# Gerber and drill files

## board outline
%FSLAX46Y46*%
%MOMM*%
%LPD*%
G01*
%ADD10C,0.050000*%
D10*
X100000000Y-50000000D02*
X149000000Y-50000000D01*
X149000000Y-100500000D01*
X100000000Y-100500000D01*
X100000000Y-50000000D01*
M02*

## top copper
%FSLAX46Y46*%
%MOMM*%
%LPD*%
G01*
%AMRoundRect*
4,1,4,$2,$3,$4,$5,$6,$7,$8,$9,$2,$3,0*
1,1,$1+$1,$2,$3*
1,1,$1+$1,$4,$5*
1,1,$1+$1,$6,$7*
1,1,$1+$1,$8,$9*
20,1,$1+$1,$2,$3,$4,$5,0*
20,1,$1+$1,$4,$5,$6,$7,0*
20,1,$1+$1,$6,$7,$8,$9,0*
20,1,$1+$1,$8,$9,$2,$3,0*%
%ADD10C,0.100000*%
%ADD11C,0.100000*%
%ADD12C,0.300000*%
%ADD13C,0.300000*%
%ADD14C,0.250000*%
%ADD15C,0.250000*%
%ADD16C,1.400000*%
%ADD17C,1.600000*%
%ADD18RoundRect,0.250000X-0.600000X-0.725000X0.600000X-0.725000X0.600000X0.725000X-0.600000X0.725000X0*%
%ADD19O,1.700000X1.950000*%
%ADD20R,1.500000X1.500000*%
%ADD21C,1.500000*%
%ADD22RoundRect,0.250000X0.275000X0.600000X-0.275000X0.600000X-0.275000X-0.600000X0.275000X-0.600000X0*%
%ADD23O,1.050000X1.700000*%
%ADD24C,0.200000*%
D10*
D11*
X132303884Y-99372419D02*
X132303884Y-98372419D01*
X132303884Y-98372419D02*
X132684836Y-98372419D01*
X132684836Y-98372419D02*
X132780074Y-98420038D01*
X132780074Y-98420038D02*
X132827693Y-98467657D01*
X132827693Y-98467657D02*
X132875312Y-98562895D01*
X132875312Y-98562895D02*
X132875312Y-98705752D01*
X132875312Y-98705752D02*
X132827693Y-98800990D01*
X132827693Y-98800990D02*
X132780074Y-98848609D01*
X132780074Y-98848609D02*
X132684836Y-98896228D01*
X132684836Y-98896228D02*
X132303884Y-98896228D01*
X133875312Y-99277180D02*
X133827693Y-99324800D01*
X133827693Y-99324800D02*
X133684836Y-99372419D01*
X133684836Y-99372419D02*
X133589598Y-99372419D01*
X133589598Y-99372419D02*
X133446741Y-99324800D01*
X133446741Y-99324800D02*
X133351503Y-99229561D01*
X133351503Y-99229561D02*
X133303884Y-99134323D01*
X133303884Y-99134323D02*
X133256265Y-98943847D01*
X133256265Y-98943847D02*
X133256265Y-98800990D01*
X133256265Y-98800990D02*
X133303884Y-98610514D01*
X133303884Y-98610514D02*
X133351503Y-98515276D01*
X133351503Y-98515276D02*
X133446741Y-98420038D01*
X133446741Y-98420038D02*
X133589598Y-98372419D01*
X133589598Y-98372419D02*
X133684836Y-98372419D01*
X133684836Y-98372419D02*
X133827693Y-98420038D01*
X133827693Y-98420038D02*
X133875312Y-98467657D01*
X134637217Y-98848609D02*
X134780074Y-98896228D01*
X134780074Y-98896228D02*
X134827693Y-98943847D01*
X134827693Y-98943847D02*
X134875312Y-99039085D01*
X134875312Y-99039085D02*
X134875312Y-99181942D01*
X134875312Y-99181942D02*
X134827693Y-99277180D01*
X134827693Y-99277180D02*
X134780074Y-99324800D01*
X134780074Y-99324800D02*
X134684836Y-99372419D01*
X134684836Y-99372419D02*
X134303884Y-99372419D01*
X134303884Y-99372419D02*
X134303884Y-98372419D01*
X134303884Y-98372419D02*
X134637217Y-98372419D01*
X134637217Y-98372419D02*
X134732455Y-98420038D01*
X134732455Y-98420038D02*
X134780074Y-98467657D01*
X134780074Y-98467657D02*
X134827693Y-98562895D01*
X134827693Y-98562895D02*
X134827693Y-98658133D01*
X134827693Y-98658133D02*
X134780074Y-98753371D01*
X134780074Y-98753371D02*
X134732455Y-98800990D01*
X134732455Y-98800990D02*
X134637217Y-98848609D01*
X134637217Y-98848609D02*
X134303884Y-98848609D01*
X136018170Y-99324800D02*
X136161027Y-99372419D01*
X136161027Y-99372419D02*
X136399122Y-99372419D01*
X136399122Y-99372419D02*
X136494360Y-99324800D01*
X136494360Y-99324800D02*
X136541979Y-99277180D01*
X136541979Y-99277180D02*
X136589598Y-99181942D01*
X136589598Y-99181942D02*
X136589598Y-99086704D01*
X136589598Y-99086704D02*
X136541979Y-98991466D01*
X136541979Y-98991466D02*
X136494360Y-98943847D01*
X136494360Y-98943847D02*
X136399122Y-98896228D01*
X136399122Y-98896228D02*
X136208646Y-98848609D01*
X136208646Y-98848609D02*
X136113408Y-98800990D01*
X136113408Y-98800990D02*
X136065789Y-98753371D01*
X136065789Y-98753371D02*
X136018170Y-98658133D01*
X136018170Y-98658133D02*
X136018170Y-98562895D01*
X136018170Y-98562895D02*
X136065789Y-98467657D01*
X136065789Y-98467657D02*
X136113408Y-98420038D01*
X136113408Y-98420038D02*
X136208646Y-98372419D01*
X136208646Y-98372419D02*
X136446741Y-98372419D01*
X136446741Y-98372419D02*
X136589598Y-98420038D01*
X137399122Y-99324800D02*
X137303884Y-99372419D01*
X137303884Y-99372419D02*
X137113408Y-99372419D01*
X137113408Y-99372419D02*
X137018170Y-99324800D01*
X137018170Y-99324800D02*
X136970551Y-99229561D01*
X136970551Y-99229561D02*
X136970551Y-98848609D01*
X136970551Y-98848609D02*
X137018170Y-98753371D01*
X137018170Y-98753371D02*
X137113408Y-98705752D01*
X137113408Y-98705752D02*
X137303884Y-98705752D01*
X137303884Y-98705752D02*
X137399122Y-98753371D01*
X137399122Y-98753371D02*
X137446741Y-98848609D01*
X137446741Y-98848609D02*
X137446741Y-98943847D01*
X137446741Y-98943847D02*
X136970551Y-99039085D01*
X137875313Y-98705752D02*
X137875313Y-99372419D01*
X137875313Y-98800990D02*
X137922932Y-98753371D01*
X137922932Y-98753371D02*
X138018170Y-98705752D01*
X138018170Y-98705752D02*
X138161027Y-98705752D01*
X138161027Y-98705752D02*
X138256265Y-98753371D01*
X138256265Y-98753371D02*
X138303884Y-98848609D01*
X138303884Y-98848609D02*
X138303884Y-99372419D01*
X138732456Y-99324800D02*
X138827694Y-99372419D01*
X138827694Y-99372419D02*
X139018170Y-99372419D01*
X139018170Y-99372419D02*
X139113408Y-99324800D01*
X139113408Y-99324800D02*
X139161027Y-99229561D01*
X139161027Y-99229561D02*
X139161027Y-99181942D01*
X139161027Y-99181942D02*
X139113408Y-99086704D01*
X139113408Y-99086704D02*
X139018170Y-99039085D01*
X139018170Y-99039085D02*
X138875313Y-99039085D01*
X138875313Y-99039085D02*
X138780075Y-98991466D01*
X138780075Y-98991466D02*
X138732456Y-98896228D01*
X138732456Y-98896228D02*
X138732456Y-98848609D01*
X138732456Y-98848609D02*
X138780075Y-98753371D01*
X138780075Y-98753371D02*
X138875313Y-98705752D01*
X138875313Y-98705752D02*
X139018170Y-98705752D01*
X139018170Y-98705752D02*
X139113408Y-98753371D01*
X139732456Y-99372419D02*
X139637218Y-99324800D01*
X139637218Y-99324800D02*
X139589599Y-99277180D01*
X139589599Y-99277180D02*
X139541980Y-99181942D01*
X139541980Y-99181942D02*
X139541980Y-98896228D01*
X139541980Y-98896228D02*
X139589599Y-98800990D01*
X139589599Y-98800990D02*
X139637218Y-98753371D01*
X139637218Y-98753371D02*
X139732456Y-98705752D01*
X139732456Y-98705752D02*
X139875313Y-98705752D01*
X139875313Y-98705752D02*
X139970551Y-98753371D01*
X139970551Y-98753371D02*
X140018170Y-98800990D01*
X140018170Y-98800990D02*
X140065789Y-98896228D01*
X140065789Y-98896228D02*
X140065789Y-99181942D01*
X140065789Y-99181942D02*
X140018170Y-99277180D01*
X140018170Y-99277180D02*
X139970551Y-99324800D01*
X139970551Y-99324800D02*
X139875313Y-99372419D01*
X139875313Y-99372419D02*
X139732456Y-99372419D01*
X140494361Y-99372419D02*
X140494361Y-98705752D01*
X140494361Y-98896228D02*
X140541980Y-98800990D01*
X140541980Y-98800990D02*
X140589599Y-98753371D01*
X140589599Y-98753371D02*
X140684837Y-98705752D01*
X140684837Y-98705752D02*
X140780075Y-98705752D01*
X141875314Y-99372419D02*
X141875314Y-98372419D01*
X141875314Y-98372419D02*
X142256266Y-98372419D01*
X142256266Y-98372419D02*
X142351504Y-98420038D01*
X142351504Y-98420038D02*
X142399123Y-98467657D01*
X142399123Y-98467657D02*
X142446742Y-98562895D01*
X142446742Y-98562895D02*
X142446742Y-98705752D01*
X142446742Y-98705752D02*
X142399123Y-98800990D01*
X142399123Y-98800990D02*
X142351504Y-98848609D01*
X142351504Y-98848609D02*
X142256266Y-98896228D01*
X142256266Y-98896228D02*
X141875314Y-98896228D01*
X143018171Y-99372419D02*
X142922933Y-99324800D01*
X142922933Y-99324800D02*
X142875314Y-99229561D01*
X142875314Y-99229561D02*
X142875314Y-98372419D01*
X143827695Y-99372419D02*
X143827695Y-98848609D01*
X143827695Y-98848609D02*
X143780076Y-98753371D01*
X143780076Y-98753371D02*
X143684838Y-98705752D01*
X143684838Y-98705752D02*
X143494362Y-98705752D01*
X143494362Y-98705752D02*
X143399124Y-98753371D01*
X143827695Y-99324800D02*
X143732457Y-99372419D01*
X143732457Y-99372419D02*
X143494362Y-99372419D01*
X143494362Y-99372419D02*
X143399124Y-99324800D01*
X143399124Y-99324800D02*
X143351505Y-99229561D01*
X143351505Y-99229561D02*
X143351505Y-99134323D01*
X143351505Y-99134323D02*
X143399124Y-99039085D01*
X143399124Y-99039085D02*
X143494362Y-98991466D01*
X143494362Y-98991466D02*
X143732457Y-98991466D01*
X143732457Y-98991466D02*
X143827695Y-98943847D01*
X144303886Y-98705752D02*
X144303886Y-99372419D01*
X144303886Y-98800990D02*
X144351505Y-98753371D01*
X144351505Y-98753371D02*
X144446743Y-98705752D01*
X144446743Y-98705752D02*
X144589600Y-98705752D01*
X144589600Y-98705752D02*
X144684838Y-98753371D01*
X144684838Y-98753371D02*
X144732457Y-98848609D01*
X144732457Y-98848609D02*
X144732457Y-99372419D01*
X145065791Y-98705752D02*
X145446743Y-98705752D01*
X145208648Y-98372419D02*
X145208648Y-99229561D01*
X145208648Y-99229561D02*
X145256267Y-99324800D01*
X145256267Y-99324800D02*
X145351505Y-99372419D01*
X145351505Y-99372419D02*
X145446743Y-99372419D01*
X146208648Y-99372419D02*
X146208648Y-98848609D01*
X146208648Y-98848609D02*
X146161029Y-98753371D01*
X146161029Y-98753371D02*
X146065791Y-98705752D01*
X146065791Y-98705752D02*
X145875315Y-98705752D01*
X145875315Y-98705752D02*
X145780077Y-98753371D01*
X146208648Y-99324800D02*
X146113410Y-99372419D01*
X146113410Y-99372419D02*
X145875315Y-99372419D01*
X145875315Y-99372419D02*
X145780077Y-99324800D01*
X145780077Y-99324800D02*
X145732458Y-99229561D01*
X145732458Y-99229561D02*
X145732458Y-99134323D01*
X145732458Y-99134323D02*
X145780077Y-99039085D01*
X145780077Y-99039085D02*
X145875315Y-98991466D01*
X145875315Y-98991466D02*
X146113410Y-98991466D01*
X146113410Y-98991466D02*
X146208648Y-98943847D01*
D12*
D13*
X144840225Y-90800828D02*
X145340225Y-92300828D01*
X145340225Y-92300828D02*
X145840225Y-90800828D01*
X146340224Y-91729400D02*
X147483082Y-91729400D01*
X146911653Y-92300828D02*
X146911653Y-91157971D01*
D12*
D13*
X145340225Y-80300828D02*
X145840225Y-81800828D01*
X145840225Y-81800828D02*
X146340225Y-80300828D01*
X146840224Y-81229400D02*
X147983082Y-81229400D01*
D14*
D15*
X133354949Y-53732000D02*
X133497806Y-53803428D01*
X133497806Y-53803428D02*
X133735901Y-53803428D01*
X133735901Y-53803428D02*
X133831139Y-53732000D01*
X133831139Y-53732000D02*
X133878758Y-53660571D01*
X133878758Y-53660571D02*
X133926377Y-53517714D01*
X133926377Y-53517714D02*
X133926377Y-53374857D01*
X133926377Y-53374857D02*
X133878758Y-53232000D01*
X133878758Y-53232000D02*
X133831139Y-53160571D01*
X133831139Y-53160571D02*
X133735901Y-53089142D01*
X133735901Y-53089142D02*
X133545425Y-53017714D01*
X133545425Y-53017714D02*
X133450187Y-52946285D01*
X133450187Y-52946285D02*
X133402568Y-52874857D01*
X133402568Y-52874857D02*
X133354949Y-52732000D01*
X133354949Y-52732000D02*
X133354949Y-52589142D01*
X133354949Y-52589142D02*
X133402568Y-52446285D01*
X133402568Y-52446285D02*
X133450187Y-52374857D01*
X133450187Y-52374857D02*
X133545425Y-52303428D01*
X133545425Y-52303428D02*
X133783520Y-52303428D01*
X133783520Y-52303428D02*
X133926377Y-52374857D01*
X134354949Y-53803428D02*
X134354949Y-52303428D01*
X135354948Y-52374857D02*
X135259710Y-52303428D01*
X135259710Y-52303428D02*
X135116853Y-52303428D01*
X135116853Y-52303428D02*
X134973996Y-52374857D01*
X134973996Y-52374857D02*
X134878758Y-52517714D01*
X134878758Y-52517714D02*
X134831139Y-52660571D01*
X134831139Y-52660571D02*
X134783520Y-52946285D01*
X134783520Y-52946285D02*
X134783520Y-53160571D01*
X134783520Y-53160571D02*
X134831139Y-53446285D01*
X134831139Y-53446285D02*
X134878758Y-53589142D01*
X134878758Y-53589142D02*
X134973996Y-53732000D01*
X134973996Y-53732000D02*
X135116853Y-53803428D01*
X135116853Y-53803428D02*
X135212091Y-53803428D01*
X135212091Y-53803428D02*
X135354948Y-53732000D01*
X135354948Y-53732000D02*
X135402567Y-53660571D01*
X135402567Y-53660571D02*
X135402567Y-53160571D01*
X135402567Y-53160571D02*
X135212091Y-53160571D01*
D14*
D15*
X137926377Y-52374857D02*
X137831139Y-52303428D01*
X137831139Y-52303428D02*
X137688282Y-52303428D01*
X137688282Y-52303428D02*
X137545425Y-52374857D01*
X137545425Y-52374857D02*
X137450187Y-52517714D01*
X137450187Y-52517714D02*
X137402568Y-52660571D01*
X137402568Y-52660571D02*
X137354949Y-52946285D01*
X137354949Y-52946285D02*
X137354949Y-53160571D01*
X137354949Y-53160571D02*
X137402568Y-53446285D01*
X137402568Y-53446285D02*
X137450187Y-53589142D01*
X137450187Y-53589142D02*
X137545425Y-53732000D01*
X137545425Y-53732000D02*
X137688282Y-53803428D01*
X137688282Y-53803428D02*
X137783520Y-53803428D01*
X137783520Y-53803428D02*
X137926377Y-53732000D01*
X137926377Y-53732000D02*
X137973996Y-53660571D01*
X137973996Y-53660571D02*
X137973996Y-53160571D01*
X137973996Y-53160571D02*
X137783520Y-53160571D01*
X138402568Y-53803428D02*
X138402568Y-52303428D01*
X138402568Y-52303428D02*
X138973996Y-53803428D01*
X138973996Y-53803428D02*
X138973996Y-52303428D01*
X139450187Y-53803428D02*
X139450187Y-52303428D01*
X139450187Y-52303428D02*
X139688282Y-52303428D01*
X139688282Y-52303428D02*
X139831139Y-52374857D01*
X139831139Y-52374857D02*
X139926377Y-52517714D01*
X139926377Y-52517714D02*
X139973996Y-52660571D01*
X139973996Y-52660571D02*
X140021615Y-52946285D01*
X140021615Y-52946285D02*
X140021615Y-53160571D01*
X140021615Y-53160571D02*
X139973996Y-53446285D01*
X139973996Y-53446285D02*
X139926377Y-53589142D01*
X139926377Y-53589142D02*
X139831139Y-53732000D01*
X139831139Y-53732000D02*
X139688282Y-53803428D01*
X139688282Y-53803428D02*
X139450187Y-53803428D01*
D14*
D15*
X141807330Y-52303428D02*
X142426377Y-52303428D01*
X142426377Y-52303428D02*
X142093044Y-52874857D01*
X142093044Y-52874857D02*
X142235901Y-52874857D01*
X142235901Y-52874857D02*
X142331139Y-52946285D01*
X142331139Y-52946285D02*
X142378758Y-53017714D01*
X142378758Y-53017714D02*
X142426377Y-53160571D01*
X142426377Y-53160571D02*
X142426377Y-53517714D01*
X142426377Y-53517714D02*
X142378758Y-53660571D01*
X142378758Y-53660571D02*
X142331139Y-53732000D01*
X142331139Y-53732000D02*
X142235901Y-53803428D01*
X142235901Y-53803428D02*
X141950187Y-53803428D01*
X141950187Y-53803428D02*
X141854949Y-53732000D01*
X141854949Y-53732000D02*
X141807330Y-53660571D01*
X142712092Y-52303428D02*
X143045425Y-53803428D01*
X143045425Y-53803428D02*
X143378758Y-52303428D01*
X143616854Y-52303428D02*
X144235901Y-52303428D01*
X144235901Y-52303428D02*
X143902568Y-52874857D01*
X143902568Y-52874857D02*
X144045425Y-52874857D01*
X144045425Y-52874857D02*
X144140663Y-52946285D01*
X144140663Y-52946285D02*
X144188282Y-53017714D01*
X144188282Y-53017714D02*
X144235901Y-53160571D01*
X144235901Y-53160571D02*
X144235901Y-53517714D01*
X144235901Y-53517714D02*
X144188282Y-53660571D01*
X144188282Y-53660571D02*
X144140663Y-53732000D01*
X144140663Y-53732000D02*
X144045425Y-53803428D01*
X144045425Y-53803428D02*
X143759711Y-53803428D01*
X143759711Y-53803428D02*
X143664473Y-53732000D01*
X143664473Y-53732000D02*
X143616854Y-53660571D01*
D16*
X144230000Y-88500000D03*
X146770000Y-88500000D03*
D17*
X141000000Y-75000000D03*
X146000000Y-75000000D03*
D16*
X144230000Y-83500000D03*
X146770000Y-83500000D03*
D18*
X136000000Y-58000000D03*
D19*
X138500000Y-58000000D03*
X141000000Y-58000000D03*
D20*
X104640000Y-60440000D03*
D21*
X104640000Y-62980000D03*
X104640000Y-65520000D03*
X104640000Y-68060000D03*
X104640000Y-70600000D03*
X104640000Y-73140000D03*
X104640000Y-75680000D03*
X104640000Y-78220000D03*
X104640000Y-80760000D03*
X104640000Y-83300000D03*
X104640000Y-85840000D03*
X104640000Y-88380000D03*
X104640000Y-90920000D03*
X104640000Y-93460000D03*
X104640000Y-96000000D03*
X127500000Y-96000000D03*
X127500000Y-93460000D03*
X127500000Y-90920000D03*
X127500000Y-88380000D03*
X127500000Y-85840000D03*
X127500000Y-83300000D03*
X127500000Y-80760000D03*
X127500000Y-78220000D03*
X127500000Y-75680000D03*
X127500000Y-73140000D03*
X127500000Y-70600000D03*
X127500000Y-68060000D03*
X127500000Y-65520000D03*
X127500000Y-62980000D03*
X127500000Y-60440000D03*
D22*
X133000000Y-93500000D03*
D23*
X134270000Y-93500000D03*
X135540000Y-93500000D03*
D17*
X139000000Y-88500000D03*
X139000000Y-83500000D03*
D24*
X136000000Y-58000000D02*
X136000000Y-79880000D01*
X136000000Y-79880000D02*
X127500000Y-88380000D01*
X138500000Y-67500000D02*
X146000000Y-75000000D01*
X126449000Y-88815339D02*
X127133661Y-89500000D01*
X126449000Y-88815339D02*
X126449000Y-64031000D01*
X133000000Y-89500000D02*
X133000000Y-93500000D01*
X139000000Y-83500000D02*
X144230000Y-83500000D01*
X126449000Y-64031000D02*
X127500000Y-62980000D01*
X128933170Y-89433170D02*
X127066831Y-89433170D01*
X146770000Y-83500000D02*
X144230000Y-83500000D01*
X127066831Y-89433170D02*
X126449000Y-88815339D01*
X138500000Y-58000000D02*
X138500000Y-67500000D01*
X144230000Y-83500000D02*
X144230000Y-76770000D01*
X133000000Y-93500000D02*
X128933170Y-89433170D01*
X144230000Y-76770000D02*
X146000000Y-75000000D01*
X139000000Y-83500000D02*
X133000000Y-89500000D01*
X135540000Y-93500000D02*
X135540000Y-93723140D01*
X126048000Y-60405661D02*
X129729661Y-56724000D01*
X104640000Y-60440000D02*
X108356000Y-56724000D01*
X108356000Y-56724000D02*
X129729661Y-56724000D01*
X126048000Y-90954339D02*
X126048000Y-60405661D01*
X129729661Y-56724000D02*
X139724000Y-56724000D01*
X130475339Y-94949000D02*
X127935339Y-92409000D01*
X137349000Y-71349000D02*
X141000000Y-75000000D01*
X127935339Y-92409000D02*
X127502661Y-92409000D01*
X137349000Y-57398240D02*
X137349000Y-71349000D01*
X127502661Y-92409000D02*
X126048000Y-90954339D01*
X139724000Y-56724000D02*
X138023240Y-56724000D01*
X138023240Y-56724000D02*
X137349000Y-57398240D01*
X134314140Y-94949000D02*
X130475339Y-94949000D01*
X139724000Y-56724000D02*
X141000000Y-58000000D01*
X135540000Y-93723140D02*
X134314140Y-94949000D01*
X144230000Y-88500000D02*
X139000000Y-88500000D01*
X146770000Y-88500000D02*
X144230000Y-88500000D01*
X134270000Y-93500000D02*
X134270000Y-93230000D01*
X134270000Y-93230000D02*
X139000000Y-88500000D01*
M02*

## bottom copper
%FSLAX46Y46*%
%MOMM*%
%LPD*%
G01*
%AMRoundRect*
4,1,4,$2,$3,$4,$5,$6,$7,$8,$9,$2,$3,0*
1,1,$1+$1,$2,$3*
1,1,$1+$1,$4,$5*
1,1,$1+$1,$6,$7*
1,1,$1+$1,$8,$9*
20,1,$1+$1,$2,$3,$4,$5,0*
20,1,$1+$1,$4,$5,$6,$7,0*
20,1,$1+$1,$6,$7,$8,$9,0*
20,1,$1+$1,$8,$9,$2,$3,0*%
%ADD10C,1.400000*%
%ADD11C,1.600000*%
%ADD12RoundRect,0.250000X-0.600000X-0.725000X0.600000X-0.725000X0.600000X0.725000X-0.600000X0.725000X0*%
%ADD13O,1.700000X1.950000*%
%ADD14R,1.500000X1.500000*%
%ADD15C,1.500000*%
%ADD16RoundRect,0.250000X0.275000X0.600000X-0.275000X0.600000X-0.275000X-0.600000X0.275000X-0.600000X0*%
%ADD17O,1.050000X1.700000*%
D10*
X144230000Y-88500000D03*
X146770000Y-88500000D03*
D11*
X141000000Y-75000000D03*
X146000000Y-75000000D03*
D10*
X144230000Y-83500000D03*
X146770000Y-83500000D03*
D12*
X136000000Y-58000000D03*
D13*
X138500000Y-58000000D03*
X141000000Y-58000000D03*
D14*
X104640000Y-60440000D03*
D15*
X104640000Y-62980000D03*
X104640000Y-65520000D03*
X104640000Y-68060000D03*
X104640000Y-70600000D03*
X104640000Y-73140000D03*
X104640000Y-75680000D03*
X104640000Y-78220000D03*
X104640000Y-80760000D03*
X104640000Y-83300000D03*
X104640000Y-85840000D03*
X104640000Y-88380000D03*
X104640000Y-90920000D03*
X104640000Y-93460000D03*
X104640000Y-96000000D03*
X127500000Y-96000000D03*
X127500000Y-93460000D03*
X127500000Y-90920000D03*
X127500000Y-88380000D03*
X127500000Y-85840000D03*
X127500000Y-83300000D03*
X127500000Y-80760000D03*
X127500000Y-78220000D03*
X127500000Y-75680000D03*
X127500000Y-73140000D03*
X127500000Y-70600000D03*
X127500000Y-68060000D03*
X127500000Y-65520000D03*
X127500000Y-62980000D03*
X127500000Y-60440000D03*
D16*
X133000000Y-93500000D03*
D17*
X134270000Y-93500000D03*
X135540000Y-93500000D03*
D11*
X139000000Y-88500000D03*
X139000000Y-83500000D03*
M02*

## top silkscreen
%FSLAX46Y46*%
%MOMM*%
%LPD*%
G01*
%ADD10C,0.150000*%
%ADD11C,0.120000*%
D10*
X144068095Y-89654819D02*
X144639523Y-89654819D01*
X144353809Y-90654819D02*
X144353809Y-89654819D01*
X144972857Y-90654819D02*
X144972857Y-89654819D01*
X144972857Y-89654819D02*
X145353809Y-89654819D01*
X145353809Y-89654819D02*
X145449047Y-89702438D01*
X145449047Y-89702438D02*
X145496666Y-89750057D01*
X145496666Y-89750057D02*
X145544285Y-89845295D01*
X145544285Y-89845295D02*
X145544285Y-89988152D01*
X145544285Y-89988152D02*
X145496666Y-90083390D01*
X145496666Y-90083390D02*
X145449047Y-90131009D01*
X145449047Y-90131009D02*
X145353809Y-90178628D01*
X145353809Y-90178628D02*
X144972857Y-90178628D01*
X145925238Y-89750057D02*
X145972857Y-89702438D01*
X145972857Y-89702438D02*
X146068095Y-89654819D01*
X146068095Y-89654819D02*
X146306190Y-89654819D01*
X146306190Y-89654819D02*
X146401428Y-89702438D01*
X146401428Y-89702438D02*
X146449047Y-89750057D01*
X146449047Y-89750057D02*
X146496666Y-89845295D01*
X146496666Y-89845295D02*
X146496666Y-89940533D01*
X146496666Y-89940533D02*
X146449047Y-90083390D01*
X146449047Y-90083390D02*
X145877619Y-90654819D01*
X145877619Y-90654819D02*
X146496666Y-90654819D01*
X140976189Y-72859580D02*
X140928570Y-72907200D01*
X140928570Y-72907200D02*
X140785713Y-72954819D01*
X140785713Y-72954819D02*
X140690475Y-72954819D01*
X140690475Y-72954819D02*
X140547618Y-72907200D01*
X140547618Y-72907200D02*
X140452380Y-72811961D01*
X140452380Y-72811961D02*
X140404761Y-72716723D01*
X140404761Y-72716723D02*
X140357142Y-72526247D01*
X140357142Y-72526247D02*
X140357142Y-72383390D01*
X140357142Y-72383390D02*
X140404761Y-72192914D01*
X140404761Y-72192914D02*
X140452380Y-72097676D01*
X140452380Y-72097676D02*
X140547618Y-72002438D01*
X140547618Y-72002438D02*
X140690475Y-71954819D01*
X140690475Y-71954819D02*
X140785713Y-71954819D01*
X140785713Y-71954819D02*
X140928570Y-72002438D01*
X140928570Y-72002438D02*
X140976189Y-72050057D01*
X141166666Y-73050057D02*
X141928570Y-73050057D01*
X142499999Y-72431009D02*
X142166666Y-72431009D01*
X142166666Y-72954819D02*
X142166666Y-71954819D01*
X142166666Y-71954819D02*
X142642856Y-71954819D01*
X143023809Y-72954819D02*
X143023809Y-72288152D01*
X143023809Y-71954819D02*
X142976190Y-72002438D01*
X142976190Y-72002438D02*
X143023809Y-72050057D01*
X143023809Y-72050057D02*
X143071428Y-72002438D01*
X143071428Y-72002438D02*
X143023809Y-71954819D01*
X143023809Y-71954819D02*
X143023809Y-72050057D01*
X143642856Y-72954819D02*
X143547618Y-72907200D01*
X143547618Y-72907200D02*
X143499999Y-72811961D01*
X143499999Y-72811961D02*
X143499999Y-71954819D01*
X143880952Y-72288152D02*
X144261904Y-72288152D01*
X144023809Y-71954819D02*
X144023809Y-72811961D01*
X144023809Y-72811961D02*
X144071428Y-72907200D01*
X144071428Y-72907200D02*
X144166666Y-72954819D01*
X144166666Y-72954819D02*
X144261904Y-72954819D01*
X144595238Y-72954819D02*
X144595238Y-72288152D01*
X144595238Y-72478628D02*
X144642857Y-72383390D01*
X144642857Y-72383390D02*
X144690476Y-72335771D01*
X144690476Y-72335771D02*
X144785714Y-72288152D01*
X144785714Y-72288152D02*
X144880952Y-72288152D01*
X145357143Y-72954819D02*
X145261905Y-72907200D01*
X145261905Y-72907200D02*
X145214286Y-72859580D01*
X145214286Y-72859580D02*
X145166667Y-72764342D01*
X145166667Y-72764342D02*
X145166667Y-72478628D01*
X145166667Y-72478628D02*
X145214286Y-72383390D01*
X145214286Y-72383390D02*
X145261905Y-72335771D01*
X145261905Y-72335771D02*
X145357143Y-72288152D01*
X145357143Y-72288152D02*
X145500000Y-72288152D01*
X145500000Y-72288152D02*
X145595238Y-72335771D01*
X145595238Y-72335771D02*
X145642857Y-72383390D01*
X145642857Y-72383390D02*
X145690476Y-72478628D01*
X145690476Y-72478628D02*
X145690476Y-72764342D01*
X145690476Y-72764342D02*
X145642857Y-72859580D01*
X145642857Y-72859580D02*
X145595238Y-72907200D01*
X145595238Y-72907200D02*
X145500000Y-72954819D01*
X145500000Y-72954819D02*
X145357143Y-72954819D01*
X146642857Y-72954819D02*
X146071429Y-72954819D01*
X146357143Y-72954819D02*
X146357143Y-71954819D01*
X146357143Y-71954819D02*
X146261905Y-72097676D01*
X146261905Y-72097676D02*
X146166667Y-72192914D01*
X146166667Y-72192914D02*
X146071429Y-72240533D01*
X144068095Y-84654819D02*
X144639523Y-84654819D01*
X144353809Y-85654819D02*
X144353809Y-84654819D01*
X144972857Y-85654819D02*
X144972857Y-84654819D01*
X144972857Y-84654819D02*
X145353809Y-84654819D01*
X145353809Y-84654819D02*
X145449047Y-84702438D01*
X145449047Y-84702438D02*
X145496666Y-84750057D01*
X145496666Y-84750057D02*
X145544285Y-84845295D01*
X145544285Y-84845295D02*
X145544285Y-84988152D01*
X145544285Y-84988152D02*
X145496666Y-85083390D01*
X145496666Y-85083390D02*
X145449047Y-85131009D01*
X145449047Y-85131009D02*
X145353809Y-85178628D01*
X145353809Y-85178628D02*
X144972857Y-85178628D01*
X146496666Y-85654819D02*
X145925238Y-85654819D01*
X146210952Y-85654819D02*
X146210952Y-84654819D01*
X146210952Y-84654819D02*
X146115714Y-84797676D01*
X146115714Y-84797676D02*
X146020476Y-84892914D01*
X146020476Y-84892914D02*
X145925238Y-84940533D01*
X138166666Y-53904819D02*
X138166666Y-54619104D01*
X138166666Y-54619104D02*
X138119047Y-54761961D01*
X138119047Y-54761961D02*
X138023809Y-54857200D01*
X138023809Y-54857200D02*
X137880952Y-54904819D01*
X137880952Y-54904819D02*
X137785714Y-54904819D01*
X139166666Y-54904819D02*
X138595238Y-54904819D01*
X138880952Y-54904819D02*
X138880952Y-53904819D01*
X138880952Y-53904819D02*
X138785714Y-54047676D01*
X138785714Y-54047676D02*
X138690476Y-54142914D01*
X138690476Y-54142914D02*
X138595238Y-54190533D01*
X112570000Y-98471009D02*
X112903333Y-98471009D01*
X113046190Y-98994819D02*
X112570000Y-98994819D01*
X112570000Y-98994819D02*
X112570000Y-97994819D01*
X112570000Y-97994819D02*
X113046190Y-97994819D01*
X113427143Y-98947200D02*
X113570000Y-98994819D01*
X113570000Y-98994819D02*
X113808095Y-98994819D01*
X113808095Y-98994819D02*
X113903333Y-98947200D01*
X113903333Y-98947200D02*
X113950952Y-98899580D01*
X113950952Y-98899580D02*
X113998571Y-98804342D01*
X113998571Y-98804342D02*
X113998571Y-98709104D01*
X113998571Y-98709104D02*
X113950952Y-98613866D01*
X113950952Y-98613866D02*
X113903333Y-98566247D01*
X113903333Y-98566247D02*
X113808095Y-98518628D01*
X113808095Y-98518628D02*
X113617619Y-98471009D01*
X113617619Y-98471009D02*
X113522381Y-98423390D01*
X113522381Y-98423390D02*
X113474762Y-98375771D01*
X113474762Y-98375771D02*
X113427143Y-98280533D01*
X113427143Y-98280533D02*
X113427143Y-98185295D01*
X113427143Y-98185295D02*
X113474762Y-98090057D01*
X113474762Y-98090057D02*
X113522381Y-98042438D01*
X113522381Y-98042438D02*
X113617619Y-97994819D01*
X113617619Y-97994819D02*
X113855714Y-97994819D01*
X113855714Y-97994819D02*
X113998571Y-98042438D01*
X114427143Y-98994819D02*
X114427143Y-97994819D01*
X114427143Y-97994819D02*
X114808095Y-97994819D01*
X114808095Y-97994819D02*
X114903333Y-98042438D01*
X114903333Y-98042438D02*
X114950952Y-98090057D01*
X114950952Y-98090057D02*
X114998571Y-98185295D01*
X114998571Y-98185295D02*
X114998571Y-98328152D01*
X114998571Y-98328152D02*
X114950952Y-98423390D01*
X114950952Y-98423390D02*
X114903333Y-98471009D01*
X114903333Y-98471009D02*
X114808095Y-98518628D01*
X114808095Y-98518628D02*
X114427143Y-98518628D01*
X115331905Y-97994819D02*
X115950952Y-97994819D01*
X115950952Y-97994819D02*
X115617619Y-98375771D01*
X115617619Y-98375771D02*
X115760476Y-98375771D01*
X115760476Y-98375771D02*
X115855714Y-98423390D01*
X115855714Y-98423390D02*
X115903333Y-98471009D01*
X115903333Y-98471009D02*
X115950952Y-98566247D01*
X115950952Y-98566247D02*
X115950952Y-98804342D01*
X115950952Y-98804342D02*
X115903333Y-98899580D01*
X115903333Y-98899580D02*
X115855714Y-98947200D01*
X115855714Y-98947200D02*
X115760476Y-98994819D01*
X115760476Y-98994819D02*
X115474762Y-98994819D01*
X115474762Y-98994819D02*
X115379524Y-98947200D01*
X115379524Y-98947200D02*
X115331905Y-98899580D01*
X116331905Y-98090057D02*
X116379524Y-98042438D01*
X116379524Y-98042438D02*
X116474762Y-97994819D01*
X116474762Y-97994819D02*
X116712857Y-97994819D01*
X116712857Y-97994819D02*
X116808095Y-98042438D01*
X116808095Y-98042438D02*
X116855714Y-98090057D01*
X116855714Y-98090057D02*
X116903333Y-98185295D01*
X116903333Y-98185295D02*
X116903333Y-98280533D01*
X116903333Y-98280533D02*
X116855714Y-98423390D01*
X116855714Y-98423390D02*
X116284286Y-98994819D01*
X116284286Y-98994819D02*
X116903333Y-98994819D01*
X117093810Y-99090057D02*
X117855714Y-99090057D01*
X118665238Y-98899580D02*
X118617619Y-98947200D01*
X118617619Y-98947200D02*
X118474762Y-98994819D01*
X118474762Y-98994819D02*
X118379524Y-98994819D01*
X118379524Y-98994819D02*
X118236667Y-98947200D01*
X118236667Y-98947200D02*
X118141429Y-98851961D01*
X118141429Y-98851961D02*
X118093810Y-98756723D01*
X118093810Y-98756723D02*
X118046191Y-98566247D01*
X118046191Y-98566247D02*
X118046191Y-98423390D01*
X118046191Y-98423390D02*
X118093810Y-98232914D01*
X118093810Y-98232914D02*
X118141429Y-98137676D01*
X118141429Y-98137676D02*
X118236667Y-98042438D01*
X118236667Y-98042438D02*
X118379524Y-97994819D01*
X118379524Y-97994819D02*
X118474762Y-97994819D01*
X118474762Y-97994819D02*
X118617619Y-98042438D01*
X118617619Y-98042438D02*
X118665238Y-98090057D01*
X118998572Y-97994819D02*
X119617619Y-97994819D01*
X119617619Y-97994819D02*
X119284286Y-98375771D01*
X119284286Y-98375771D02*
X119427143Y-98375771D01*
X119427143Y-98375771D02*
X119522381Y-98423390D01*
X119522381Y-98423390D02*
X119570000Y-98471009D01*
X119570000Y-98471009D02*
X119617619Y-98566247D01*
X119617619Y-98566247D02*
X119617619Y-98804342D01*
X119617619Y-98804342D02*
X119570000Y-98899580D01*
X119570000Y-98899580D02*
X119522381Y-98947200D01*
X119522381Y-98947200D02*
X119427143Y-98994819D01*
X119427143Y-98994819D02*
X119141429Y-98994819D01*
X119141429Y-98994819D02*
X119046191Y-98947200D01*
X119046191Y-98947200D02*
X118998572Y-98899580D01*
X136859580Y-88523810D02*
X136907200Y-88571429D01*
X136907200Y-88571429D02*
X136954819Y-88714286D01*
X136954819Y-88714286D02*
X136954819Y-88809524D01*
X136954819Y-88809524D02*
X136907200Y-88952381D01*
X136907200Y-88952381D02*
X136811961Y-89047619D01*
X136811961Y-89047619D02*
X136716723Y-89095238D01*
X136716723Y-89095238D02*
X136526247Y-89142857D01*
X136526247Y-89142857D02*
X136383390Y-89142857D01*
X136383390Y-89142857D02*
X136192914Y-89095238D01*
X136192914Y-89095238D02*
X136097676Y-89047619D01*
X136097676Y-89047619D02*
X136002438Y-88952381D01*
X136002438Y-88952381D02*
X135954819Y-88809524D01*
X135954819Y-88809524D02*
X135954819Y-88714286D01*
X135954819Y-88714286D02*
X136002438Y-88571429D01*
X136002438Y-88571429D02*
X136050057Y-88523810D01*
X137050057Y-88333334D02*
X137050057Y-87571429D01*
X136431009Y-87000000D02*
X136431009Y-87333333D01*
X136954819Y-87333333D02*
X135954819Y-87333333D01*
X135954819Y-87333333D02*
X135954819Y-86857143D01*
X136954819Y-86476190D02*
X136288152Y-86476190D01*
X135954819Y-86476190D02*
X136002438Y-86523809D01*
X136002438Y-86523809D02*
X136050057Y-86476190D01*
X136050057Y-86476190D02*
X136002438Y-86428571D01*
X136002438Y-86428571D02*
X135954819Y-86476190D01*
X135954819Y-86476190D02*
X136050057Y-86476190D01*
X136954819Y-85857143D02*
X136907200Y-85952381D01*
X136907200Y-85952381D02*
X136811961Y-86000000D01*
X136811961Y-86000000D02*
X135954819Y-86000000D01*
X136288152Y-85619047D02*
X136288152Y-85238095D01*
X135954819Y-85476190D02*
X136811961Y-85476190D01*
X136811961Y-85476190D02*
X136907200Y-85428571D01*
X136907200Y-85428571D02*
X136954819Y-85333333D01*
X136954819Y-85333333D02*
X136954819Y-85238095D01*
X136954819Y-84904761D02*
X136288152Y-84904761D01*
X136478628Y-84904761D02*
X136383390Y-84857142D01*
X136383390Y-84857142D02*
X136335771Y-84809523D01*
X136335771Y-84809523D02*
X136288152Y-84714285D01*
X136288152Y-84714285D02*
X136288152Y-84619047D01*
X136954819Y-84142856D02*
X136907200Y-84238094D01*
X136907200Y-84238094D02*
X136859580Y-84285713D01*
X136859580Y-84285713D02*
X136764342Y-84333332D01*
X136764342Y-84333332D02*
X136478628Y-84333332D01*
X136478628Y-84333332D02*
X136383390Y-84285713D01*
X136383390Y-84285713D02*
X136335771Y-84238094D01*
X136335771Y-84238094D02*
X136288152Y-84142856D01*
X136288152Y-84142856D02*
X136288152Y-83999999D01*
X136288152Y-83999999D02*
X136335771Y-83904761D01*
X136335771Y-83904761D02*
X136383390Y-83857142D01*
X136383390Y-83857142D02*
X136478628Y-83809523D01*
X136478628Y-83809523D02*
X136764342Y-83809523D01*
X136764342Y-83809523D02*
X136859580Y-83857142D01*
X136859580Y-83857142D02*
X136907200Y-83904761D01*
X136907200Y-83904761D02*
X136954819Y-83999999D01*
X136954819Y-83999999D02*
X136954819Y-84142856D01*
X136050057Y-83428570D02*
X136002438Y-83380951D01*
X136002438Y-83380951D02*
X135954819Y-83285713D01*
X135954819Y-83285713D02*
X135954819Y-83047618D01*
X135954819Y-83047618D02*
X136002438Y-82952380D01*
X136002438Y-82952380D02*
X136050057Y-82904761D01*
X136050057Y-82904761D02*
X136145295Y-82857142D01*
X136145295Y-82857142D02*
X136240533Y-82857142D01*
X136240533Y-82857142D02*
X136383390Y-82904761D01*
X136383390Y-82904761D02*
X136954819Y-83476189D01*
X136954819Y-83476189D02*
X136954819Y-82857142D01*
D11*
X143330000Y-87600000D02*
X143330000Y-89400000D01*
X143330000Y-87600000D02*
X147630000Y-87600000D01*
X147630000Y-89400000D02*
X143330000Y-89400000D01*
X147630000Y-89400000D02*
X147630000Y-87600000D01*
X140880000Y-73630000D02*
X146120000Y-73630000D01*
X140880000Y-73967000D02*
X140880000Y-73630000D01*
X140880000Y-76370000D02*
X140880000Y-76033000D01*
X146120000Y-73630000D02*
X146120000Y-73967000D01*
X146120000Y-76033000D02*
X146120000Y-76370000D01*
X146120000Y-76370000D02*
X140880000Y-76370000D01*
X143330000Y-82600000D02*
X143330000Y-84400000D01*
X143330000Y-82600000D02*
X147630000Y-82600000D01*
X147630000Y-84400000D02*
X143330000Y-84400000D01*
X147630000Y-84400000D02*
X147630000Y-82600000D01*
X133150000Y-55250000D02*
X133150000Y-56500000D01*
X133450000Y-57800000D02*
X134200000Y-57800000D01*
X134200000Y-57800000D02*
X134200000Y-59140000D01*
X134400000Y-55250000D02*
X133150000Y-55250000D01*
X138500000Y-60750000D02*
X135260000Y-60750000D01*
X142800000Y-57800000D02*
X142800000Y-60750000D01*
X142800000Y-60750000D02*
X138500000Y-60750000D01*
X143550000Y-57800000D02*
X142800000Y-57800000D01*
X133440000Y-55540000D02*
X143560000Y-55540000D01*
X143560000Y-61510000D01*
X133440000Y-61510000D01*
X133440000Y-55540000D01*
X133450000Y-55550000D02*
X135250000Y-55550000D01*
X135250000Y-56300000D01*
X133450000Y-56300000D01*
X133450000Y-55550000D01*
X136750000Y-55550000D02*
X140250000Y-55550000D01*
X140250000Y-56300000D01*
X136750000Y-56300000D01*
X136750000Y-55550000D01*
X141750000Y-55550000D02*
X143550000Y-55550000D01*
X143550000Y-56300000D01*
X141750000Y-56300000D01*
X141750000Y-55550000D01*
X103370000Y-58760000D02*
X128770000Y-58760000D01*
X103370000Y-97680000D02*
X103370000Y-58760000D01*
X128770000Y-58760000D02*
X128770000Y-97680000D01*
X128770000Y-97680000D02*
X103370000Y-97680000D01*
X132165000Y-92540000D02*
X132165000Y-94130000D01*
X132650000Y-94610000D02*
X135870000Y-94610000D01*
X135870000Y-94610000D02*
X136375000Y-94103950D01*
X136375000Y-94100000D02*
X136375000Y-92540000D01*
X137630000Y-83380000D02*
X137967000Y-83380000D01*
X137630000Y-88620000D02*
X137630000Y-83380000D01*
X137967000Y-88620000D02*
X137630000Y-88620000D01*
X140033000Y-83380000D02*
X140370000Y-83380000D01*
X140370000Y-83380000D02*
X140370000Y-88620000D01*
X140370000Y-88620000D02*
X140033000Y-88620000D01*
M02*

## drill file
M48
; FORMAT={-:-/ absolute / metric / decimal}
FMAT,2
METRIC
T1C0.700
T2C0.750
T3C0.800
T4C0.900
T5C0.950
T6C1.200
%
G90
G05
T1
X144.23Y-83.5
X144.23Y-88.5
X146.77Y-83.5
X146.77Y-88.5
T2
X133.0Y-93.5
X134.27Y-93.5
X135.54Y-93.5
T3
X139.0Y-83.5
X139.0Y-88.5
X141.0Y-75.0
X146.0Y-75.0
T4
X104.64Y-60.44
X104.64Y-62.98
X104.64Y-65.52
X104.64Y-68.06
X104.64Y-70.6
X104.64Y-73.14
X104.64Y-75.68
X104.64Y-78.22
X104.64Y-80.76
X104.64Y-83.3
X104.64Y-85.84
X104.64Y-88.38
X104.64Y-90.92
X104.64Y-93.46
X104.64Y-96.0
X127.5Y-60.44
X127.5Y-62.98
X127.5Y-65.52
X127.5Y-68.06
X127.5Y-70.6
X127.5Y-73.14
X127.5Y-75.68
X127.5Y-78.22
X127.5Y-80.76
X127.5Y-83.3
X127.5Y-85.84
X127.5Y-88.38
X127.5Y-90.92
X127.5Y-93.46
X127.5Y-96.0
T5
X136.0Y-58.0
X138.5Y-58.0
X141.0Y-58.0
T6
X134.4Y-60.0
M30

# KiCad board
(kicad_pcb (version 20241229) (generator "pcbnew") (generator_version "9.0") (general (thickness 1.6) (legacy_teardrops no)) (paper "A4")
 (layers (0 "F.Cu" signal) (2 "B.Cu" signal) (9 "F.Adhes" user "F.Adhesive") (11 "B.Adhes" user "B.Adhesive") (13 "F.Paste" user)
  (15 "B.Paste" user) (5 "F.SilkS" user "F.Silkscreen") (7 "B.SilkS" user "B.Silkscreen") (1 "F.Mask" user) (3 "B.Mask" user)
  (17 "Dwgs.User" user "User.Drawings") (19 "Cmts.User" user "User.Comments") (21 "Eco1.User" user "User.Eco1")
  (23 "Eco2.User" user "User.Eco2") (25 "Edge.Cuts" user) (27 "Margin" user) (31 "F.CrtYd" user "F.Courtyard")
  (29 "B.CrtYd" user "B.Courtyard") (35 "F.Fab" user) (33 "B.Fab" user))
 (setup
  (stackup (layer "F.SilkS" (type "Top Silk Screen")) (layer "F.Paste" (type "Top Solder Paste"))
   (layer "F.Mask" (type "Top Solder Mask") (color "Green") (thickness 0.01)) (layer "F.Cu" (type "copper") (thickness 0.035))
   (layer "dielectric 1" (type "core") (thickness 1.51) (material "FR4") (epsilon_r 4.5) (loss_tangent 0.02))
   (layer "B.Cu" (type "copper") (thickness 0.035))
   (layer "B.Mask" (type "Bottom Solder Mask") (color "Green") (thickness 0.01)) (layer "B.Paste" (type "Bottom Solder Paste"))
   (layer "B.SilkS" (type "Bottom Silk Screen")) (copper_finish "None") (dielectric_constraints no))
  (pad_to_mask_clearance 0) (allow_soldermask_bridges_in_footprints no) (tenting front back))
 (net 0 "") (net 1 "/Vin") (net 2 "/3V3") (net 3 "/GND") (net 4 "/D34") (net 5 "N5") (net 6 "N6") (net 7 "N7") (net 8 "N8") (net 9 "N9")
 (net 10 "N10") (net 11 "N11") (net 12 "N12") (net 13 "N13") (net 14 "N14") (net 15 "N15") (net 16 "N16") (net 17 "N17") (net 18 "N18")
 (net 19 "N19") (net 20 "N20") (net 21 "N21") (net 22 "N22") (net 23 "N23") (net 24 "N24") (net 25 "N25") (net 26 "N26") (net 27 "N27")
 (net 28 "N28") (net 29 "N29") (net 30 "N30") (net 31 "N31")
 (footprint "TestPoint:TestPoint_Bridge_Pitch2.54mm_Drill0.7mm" (layer "F.Cu") (at 144.23 88.5)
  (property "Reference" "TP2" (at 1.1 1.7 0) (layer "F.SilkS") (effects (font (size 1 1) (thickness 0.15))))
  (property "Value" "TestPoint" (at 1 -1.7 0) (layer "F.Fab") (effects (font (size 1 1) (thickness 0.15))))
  (fp_line (start -0.9 -0.9) (end -0.9 0.9) (stroke (width 0.12) (type solid)) (layer "F.SilkS"))
  (fp_line (start -0.9 -0.9) (end 3.4 -0.9) (stroke (width 0.12) (type solid)) (layer "F.SilkS"))
  (fp_line (start 3.4 0.9) (end -0.9 0.9) (stroke (width 0.12) (type solid)) (layer "F.SilkS"))
  (fp_line (start 3.4 0.9) (end 3.4 -0.9) (stroke (width 0.12) (type solid)) (layer "F.SilkS"))
  (pad "1" thru_hole circle (at 0 0) (size 1.4 1.4) (drill 0.7) (layers "*.Cu" "*.Mask") (remove_unused_layers no) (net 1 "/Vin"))
  (pad "1" thru_hole circle (at 2.54 0) (size 1.4 1.4) (drill 0.7) (layers "*.Cu" "*.Mask") (remove_unused_layers no) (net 1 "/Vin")))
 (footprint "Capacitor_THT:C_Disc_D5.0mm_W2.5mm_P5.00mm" (layer "F.Cu") (at 141 75)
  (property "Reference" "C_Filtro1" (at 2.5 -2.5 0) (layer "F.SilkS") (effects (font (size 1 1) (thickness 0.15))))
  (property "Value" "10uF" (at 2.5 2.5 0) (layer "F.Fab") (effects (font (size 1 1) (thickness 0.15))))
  (fp_line (start -0.12 -1.37) (end 5.12 -1.37) (stroke (width 0.12) (type solid)) (layer "F.SilkS"))
  (fp_line (start -0.12 -1.033) (end -0.12 -1.37) (stroke (width 0.12) (type solid)) (layer "F.SilkS"))
  (fp_line (start -0.12 1.37) (end -0.12 1.033) (stroke (width 0.12) (type solid)) (layer "F.SilkS"))
  (fp_line (start 5.12 -1.37) (end 5.12 -1.033) (stroke (width 0.12) (type solid)) (layer "F.SilkS"))
  (fp_line (start 5.12 1.033) (end 5.12 1.37) (stroke (width 0.12) (type solid)) (layer "F.SilkS"))
  (fp_line (start 5.12 1.37) (end -0.12 1.37) (stroke (width 0.12) (type solid)) (layer "F.SilkS"))
  (pad "1" thru_hole circle (at 0 0) (size 1.6 1.6) (drill 0.8) (layers "*.Cu" "*.Mask") (remove_unused_layers no) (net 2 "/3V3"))
  (pad "2" thru_hole circle (at 5 0) (size 1.6 1.6) (drill 0.8) (layers "*.Cu" "*.Mask") (remove_unused_layers no) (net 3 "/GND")))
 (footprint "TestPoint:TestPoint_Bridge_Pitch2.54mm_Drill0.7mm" (layer "F.Cu") (at 144.23 83.5)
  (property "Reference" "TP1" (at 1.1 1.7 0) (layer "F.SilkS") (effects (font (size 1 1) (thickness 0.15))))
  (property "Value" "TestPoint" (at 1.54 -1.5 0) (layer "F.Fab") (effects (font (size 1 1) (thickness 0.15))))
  (fp_line (start -0.9 -0.9) (end -0.9 0.9) (stroke (width 0.12) (type solid)) (layer "F.SilkS"))
  (fp_line (start -0.9 -0.9) (end 3.4 -0.9) (stroke (width 0.12) (type solid)) (layer "F.SilkS"))
  (fp_line (start 3.4 0.9) (end -0.9 0.9) (stroke (width 0.12) (type solid)) (layer "F.SilkS"))
  (fp_line (start 3.4 0.9) (end 3.4 -0.9) (stroke (width 0.12) (type solid)) (layer "F.SilkS"))
  (pad "1" thru_hole circle (at 0 0) (size 1.4 1.4) (drill 0.7) (layers "*.Cu" "*.Mask") (remove_unused_layers no) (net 3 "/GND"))
  (pad "1" thru_hole circle (at 2.54 0) (size 1.4 1.4) (drill 0.7) (layers "*.Cu" "*.Mask") (remove_unused_layers no) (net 3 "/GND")))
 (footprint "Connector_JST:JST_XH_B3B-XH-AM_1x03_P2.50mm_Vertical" (layer "F.Cu") (at 136 58)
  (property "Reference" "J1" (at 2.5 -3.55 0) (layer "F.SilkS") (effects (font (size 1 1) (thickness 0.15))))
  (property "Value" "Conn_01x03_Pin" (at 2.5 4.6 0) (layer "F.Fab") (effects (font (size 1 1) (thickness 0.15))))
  (fp_line (start -2.85 -2.75) (end -2.85 -1.5) (stroke (width 0.12) (type solid)) (layer "F.SilkS"))
  (fp_line (start -2.55 -0.2) (end -1.8 -0.2) (stroke (width 0.12) (type solid)) (layer "F.SilkS"))
  (fp_line (start -1.8 -0.2) (end -1.8 1.14) (stroke (width 0.12) (type solid)) (layer "F.SilkS"))
  (fp_line (start -1.6 -2.75) (end -2.85 -2.75) (stroke (width 0.12) (type solid)) (layer "F.SilkS"))
  (fp_line (start 2.5 2.75) (end -0.74 2.75) (stroke (width 0.12) (type solid)) (layer "F.SilkS"))
  (fp_line (start 6.8 -0.2) (end 6.8 2.75) (stroke (width 0.12) (type solid)) (layer "F.SilkS"))
  (fp_line (start 6.8 2.75) (end 2.5 2.75) (stroke (width 0.12) (type solid)) (layer "F.SilkS"))
  (fp_line (start 7.55 -0.2) (end 6.8 -0.2) (stroke (width 0.12) (type solid)) (layer "F.SilkS"))
  (fp_rect (start -2.56 -2.46) (end 7.56 3.51) (stroke (width 0.12) (type solid)) (fill no) (layer "F.SilkS"))
  (fp_rect (start -2.55 -2.45) (end -0.75 -1.7) (stroke (width 0.12) (type solid)) (fill no) (layer "F.SilkS"))
  (fp_rect (start 0.75 -2.45) (end 4.25 -1.7) (stroke (width 0.12) (type solid)) (fill no) (layer "F.SilkS"))
  (fp_rect (start 5.75 -2.45) (end 7.55 -1.7) (stroke (width 0.12) (type solid)) (fill no) (layer "F.SilkS"))
  (pad "" np_thru_hole circle (at -1.6 2) (size 1.2 1.2) (drill 1.2) (layers "*.Cu" "*.Mask"))
  (pad "1" thru_hole roundrect (at 0 0) (size 1.7 1.95) (drill 0.95) (layers "*.Cu" "*.Mask") (remove_unused_layers no)
   (roundrect_rratio 0.147059) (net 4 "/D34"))
  (pad "2" thru_hole oval (at 2.5 0) (size 1.7 1.95) (drill 0.95) (layers "*.Cu" "*.Mask") (remove_unused_layers no) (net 3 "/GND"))
  (pad "3" thru_hole oval (at 5 0) (size 1.7 1.95) (drill 0.95) (layers "*.Cu" "*.Mask") (remove_unused_layers no) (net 2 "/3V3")))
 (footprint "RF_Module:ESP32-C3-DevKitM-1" (layer "F.Cu") (at 104.64 60.44)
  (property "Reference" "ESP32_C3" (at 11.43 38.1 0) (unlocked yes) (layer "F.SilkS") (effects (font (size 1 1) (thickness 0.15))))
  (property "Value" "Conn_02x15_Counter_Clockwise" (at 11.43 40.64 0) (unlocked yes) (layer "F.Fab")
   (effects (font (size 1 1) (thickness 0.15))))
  (fp_line (start -1.27 -1.68) (end 24.13 -1.68) (stroke (width 0.12) (type solid)) (layer "F.SilkS"))
  (fp_line (start -1.27 37.24) (end -1.27 -1.68) (stroke (width 0.12) (type solid)) (layer "F.SilkS"))
  (fp_line (start 24.13 -1.68) (end 24.13 37.24) (stroke (width 0.12) (type solid)) (layer "F.SilkS"))
  (fp_line (start 24.13 37.24) (end -1.27 37.24) (stroke (width 0.12) (type solid)) (layer "F.SilkS"))
  (pad "1" thru_hole rect (at 0 0) (size 1.5 1.5) (drill 0.9) (layers "*.Cu" "*.Mask") (remove_unused_layers yes) (keep_end_layers yes)
   (zone_layer_connections) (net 2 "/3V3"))
  (pad "2" thru_hole circle (at 0 2.54) (size 1.5 1.5) (drill 0.9) (layers "*.Cu" "*.Mask") (remove_unused_layers yes) (keep_end_layers yes)
   (zone_layer_connections) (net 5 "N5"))
  (pad "3" thru_hole circle (at 0 5.08) (size 1.5 1.5) (drill 0.9) (layers "*.Cu" "*.Mask") (remove_unused_layers yes) (keep_end_layers yes)
   (zone_layer_connections) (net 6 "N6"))
  (pad "4" thru_hole circle (at 0 7.62) (size 1.5 1.5) (drill 0.9) (layers "*.Cu" "*.Mask") (remove_unused_layers yes) (keep_end_layers yes)
   (zone_layer_connections) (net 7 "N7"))
  (pad "5" thru_hole circle (at 0 10.16) (size 1.5 1.5) (drill 0.9) (layers "*.Cu" "*.Mask") (remove_unused_layers yes)
   (keep_end_layers yes) (zone_layer_connections) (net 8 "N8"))
  (pad "6" thru_hole circle (at 0 12.7) (size 1.5 1.5) (drill 0.9) (layers "*.Cu" "*.Mask") (remove_unused_layers yes) (keep_end_layers yes)
   (zone_layer_connections) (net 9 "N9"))
  (pad "7" thru_hole circle (at 0 15.24) (size 1.5 1.5) (drill 0.9) (layers "*.Cu" "*.Mask") (remove_unused_layers yes)
   (keep_end_layers yes) (zone_layer_connections) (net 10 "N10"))
  (pad "8" thru_hole circle (at 0 17.78) (size 1.5 1.5) (drill 0.9) (layers "*.Cu" "*.Mask") (remove_unused_layers yes)
   (keep_end_layers yes) (zone_layer_connections) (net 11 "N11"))
  (pad "9" thru_hole circle (at 0 20.32) (size 1.5 1.5) (drill 0.9) (layers "*.Cu" "*.Mask") (remove_unused_layers yes)
   (keep_end_layers yes) (zone_layer_connections) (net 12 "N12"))
  (pad "10" thru_hole circle (at 0 22.86) (size 1.5 1.5) (drill 0.9) (layers "*.Cu" "*.Mask") (remove_unused_layers yes)
   (keep_end_layers yes) (zone_layer_connections) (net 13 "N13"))
  (pad "11" thru_hole circle (at 0 25.4) (size 1.5 1.5) (drill 0.9) (layers "*.Cu" "*.Mask") (remove_unused_layers yes)
   (keep_end_layers yes) (zone_layer_connections) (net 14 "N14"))
  (pad "12" thru_hole circle (at 0 27.94) (size 1.5 1.5) (drill 0.9) (layers "*.Cu" "*.Mask") (remove_unused_layers yes)
   (keep_end_layers yes) (zone_layer_connections) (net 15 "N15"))
  (pad "13" thru_hole circle (at 0 30.48) (size 1.5 1.5) (drill 0.9) (layers "*.Cu" "*.Mask") (remove_unused_layers yes)
   (keep_end_layers yes) (zone_layer_connections) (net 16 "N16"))
  (pad "14" thru_hole circle (at 0 33.02) (size 1.5 1.5) (drill 0.9) (layers "*.Cu" "*.Mask") (remove_unused_layers yes)
   (keep_end_layers yes) (zone_layer_connections) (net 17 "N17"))
  (pad "15" thru_hole circle (at 0 35.56) (size 1.5 1.5) (drill 0.9) (layers "*.Cu" "*.Mask") (remove_unused_layers yes)
   (keep_end_layers yes) (zone_layer_connections) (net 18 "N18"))
  (pad "16" thru_hole circle (at 22.86 35.56) (size 1.5 1.5) (drill 0.9) (layers "*.Cu" "*.Mask") (remove_unused_layers yes)
   (keep_end_layers yes) (zone_layer_connections) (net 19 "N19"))
  (pad "17" thru_hole circle (at 22.86 33.02) (size 1.5 1.5) (drill 0.9) (layers "*.Cu" "*.Mask") (remove_unused_layers yes)
   (keep_end_layers yes) (zone_layer_connections) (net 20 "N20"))
  (pad "18" thru_hole circle (at 22.86 30.48) (size 1.5 1.5) (drill 0.9) (layers "*.Cu" "*.Mask") (remove_unused_layers yes)
   (keep_end_layers yes) (zone_layer_connections) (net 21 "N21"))
  (pad "19" thru_hole circle (at 22.86 27.94) (size 1.5 1.5) (drill 0.9) (layers "*.Cu" "*.Mask") (remove_unused_layers yes)
   (keep_end_layers yes) (zone_layer_connections) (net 4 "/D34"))
  (pad "20" thru_hole circle (at 22.86 25.4) (size 1.5 1.5) (drill 0.9) (layers "*.Cu" "*.Mask") (remove_unused_layers yes)
   (keep_end_layers yes) (zone_layer_connections) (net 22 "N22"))
  (pad "21" thru_hole circle (at 22.86 22.86) (size 1.5 1.5) (drill 0.9) (layers "*.Cu" "*.Mask") (remove_unused_layers yes)
   (keep_end_layers yes) (zone_layer_connections) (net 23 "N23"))
  (pad "22" thru_hole circle (at 22.86 20.32) (size 1.5 1.5) (drill 0.9) (layers "*.Cu" "*.Mask") (remove_unused_layers yes)
   (keep_end_layers yes) (zone_layer_connections) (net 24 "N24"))
  (pad "23" thru_hole circle (at 22.86 17.78) (size 1.5 1.5) (drill 0.9) (layers "*.Cu" "*.Mask") (remove_unused_layers yes)
   (keep_end_layers yes) (zone_layer_connections) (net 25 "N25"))
  (pad "24" thru_hole circle (at 22.86 15.24) (size 1.5 1.5) (drill 0.9) (layers "*.Cu" "*.Mask") (remove_unused_layers yes)
   (keep_end_layers yes) (zone_layer_connections) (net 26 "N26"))
  (pad "25" thru_hole circle (at 22.86 12.7) (size 1.5 1.5) (drill 0.9) (layers "*.Cu" "*.Mask") (remove_unused_layers yes)
   (keep_end_layers yes) (zone_layer_connections) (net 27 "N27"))
  (pad "26" thru_hole circle (at 22.86 10.16) (size 1.5 1.5) (drill 0.9) (layers "*.Cu" "*.Mask") (remove_unused_layers yes)
   (keep_end_layers yes) (zone_layer_connections) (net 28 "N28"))
  (pad "27" thru_hole circle (at 22.86 7.62) (size 1.5 1.5) (drill 0.9) (layers "*.Cu" "*.Mask") (remove_unused_layers yes)
   (keep_end_layers yes) (zone_layer_connections) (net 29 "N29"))
  (pad "28" thru_hole circle (at 22.86 5.08) (size 1.5 1.5) (drill 0.9) (layers "*.Cu" "*.Mask") (remove_unused_layers yes)
   (keep_end_layers yes) (zone_layer_connections) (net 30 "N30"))
  (pad "29" thru_hole circle (at 22.86 2.54) (size 1.5 1.5) (drill 0.9) (layers "*.Cu" "*.Mask") (remove_unused_layers yes)
   (keep_end_layers yes) (zone_layer_connections) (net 3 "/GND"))
  (pad "30" thru_hole circle (at 22.86 0) (size 1.5 1.5) (drill 0.9) (layers "*.Cu" "*.Mask") (remove_unused_layers yes)
   (keep_end_layers yes) (zone_layer_connections) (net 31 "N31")))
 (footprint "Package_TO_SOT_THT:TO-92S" (layer "F.Cu") (at 133 93.5)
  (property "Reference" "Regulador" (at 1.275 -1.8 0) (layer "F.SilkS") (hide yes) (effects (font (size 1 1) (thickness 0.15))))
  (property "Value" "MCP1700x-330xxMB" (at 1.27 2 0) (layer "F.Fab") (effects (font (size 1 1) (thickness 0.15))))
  (fp_line (start -0.835 -0.96) (end -0.835 0.63) (stroke (width 0.12) (type solid)) (layer "F.SilkS"))
  (fp_line (start -0.35 1.11) (end 2.87 1.11) (stroke (width 0.12) (type solid)) (layer "F.SilkS"))
  (fp_line (start 2.87 1.11) (end 3.375 0.60395) (stroke (width 0.12) (type solid)) (layer "F.SilkS"))
  (fp_line (start 3.375 0.6) (end 3.375 -0.96) (stroke (width 0.12) (type solid)) (layer "F.SilkS"))
  (pad "1" thru_hole roundrect (at 0 0 180) (size 1.05 1.7) (drill 0.75) (layers "*.Cu" "*.Mask") (remove_unused_layers no)
   (roundrect_rratio 0.2380952381) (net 3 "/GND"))
  (pad "2" thru_hole oval (at 1.27 0 180) (size 1.05 1.7) (drill 0.75) (layers "*.Cu" "*.Mask") (remove_unused_layers no) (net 1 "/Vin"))
  (pad "3" thru_hole oval (at 2.54 0 180) (size 1.05 1.7) (drill 0.75) (layers "*.Cu" "*.Mask") (remove_unused_layers no) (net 2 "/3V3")))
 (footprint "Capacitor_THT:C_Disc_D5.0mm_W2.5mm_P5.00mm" (layer "F.Cu") (at 139 88.5 90)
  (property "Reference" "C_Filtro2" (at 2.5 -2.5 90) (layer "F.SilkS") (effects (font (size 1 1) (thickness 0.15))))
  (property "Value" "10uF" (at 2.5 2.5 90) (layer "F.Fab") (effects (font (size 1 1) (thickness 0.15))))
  (fp_line (start 5.12 -1.37) (end 5.12 -1.033) (stroke (width 0.12) (type solid)) (layer "F.SilkS"))
  (fp_line (start -0.12 -1.37) (end 5.12 -1.37) (stroke (width 0.12) (type solid)) (layer "F.SilkS"))
  (fp_line (start -0.12 -1.033) (end -0.12 -1.37) (stroke (width 0.12) (type solid)) (layer "F.SilkS"))
  (fp_line (start 5.12 1.033) (end 5.12 1.37) (stroke (width 0.12) (type solid)) (layer "F.SilkS"))
  (fp_line (start 5.12 1.37) (end -0.12 1.37) (stroke (width 0.12) (type solid)) (layer "F.SilkS"))
  (fp_line (start -0.12 1.37) (end -0.12 1.033) (stroke (width 0.12) (type solid)) (layer "F.SilkS"))
  (pad "1" thru_hole circle (at 0 0 90) (size 1.6 1.6) (drill 0.8) (layers "*.Cu" "*.Mask") (remove_unused_layers no) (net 1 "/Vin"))
  (pad "2" thru_hole circle (at 5 0 90) (size 1.6 1.6) (drill 0.8) (layers "*.Cu" "*.Mask") (remove_unused_layers no) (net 3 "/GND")))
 (gr_rect (start 100 50) (end 149 100.5) (stroke (width 0.05) (type default)) (fill no) (layer "Edge.Cuts"))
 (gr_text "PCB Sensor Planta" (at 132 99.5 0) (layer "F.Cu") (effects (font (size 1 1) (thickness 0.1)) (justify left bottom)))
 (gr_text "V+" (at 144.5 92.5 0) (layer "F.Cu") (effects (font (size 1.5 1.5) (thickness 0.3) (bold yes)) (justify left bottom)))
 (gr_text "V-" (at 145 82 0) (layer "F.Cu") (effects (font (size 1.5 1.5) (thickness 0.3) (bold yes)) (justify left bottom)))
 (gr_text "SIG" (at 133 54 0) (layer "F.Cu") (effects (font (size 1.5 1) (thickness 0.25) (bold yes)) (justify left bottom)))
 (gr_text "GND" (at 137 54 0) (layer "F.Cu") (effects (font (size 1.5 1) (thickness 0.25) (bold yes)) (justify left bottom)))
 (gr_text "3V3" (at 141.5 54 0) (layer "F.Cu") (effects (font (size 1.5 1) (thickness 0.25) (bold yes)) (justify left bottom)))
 (segment (start 136 58) (end 136 79.88) (width 0.2) (layer "F.Cu") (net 4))
 (segment (start 136 79.88) (end 127.5 88.38) (width 0.2) (layer "F.Cu") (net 4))
 (segment (start 138.5 67.5) (end 146 75) (width 0.2) (layer "F.Cu") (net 3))
 (segment (start 126.449 88.815339) (end 127.133661 89.5) (width 0.2) (layer "F.Cu") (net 3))
 (segment (start 126.449 88.815339) (end 126.449 64.031) (width 0.2) (layer "F.Cu") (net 3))
 (segment (start 133 89.5) (end 133 93.5) (width 0.2) (layer "F.Cu") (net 3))
 (segment (start 139 83.5) (end 144.23 83.5) (width 0.2) (layer "F.Cu") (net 3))
 (segment (start 126.449 64.031) (end 127.5 62.98) (width 0.2) (layer "F.Cu") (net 3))
 (segment (start 128.93317 89.43317) (end 127.066831 89.43317) (width 0.2) (layer "F.Cu") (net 3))
 (segment (start 146.77 83.5) (end 144.23 83.5) (width 0.2) (layer "F.Cu") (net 3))
 (segment (start 127.066831 89.43317) (end 126.449 88.815339) (width 0.2) (layer "F.Cu") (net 3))
 (segment (start 138.5 58) (end 138.5 67.5) (width 0.2) (layer "F.Cu") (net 3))
 (segment (start 144.23 83.5) (end 144.23 76.77) (width 0.2) (layer "F.Cu") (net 3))
 (segment (start 133 93.5) (end 128.93317 89.43317) (width 0.2) (layer "F.Cu") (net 3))
 (segment (start 144.23 76.77) (end 146 75) (width 0.2) (layer "F.Cu") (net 3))
 (segment (start 139 83.5) (end 133 89.5) (width 0.2) (layer "F.Cu") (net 3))
 (segment (start 135.54 93.5) (end 135.54 93.72314) (width 0.2) (layer "F.Cu") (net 2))
 (segment (start 126.048 60.405661) (end 129.729661 56.724) (width 0.2) (layer "F.Cu") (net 2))
 (segment (start 104.64 60.44) (end 108.356 56.724) (width 0.2) (layer "F.Cu") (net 2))
 (segment (start 108.356 56.724) (end 129.729661 56.724) (width 0.2) (layer "F.Cu") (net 2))
 (segment (start 126.048 90.954339) (end 126.048 60.405661) (width 0.2) (layer "F.Cu") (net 2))
 (segment (start 129.729661 56.724) (end 139.724 56.724) (width 0.2) (layer "F.Cu") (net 2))
 (segment (start 130.475339 94.949) (end 127.935339 92.409) (width 0.2) (layer "F.Cu") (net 2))
 (segment (start 137.349 71.349) (end 141 75) (width 0.2) (layer "F.Cu") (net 2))
 (segment (start 127.935339 92.409) (end 127.502661 92.409) (width 0.2) (layer "F.Cu") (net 2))
 (segment (start 137.349 57.39824) (end 137.349 71.349) (width 0.2) (layer "F.Cu") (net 2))
 (segment (start 127.502661 92.409) (end 126.048 90.954339) (width 0.2) (layer "F.Cu") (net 2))
 (segment (start 139.724 56.724) (end 138.02324 56.724) (width 0.2) (layer "F.Cu") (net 2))
 (segment (start 138.02324 56.724) (end 137.349 57.39824) (width 0.2) (layer "F.Cu") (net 2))
 (segment (start 134.31414 94.949) (end 130.475339 94.949) (width 0.2) (layer "F.Cu") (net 2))
 (segment (start 139.724 56.724) (end 141 58) (width 0.2) (layer "F.Cu") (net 2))
 (segment (start 135.54 93.72314) (end 134.31414 94.949) (width 0.2) (layer "F.Cu") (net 2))
 (segment (start 144.23 88.5) (end 139 88.5) (width 0.2) (layer "F.Cu") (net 1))
 (segment (start 146.77 88.5) (end 144.23 88.5) (width 0.2) (layer "F.Cu") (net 1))
 (segment (start 134.27 93.5) (end 134.27 93.23) (width 0.2) (layer "F.Cu") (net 1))
 (segment (start 134.27 93.23) (end 139 88.5) (width 0.2) (layer "F.Cu") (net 1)))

